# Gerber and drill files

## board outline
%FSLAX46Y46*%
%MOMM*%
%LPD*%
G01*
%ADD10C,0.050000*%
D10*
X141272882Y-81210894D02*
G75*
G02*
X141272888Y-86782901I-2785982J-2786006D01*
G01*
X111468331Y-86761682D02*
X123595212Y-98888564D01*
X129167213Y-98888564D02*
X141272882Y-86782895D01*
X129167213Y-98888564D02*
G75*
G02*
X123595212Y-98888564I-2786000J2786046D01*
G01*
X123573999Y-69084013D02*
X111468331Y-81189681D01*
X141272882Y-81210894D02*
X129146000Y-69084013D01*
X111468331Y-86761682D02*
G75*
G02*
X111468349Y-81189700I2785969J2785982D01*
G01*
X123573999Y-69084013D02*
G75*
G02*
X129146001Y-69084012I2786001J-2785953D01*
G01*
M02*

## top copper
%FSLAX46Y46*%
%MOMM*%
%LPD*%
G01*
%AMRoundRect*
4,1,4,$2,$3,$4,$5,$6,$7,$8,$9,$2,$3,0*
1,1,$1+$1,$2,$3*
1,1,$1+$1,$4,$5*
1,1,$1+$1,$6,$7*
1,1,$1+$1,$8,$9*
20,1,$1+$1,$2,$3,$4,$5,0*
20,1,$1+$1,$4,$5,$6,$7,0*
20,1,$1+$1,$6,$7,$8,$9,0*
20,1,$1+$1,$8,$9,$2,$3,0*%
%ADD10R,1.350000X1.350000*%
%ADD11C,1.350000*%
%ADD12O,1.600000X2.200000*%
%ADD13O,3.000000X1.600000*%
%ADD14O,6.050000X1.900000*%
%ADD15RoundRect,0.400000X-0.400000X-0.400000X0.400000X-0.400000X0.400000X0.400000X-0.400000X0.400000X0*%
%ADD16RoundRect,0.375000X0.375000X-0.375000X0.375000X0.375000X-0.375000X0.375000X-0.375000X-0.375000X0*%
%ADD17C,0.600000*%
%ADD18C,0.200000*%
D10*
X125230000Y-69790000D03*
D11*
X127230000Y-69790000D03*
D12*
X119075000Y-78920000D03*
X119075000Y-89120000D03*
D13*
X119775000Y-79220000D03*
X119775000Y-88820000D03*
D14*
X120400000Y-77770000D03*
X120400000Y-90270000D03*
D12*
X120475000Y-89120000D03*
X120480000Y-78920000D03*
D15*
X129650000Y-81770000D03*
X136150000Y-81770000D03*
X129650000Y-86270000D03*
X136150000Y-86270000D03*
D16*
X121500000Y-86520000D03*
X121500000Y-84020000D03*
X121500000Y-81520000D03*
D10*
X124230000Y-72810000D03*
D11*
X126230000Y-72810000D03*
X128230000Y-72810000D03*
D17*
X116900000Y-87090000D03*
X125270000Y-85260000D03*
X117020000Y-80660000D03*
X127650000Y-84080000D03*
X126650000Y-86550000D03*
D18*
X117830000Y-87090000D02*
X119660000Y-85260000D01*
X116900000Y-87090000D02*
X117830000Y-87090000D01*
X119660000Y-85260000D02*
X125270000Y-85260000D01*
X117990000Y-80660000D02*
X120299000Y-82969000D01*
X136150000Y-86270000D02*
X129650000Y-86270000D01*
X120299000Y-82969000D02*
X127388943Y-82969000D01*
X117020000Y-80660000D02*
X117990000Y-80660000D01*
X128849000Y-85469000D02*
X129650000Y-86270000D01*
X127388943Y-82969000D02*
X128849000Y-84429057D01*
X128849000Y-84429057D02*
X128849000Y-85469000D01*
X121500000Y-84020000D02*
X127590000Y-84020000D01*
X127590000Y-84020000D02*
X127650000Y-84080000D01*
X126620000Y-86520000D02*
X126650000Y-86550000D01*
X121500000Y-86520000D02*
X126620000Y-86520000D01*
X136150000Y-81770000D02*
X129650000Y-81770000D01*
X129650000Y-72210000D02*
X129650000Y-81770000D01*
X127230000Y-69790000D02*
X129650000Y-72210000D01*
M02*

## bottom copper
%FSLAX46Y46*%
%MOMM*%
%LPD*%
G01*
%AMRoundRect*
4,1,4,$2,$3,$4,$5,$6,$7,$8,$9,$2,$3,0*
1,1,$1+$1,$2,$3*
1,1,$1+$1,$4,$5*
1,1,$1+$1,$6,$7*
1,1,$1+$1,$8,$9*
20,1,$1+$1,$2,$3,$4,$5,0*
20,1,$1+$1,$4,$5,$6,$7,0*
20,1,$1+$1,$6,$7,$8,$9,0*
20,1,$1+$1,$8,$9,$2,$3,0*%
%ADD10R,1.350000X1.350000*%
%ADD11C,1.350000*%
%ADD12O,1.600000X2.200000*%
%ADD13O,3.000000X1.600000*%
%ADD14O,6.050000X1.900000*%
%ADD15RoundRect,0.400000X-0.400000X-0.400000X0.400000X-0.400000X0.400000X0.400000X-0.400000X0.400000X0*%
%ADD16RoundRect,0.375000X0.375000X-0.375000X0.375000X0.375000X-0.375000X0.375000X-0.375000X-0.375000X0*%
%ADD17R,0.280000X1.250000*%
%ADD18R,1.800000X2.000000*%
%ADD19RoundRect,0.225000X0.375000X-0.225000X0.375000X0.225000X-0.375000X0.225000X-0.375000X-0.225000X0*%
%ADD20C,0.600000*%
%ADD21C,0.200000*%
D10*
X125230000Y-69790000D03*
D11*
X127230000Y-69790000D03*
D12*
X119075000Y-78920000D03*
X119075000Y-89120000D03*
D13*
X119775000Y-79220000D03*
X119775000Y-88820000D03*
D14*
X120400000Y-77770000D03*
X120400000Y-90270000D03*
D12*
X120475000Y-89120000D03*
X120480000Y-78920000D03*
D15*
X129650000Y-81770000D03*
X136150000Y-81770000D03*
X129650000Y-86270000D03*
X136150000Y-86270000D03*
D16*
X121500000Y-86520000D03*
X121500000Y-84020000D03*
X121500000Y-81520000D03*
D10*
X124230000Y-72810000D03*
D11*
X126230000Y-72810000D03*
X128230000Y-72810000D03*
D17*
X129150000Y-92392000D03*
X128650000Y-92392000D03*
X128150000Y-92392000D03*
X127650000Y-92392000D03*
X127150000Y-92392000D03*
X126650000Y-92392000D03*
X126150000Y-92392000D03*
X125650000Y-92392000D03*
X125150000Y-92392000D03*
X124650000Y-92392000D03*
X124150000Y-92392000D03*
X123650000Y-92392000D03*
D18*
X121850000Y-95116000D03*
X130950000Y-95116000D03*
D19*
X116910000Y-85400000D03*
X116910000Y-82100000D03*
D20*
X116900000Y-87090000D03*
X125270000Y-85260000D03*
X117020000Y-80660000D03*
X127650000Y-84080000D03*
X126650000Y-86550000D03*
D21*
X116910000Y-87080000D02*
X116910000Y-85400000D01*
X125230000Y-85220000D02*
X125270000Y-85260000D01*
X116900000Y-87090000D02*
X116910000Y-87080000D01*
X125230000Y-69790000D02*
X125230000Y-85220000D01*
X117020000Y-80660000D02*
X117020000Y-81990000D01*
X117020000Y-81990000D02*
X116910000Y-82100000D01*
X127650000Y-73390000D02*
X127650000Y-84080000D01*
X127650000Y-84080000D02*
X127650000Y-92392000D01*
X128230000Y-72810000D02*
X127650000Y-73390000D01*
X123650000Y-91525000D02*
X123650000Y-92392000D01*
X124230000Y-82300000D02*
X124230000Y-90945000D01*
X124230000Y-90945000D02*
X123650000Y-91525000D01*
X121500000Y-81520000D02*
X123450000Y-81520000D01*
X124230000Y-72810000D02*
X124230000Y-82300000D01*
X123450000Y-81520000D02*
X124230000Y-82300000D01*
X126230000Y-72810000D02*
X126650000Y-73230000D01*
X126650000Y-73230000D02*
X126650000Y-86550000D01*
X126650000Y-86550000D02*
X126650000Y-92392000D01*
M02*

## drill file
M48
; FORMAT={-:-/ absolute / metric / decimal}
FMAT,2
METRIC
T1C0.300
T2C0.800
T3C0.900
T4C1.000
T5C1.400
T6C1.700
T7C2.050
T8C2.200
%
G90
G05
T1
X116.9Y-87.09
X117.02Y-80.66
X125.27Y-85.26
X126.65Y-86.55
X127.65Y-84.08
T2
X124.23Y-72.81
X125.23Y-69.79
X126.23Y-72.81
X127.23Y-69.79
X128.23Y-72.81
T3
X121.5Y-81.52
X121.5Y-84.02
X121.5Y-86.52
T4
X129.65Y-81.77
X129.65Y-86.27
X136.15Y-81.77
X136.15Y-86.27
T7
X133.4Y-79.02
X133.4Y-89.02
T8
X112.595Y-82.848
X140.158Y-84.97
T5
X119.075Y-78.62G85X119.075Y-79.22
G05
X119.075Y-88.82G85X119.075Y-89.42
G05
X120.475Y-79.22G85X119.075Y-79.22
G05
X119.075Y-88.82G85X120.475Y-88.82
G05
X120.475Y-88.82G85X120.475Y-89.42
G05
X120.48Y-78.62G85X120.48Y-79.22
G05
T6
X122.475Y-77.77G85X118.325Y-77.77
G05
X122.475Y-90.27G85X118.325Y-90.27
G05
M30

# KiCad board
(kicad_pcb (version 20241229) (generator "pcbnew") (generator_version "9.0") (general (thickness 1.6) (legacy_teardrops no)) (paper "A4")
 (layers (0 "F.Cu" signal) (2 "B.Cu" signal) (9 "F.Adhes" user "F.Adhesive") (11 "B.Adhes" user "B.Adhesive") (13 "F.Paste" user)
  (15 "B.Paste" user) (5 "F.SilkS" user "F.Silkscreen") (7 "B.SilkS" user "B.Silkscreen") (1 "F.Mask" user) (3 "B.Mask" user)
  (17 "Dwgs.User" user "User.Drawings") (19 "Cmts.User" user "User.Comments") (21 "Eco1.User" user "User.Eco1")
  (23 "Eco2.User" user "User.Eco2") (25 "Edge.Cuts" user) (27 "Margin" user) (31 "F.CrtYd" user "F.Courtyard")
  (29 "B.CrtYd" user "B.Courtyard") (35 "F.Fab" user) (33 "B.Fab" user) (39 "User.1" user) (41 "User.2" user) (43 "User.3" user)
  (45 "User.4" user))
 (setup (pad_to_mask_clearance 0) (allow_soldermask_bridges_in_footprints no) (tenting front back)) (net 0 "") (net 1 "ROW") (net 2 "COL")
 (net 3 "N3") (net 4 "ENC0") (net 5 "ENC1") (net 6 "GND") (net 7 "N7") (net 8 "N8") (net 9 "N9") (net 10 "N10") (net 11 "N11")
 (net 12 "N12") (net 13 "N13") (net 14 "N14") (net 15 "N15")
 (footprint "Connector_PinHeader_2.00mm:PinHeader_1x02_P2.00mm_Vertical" (layer "F.Cu") (at 125.23 69.79 90)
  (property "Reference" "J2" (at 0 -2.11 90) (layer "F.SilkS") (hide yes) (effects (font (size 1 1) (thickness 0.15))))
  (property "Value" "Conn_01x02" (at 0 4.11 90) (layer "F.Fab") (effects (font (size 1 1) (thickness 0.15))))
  (pad "1" thru_hole rect (at 0 0 90) (size 1.35 1.35) (drill 0.8) (layers "*.Cu" "*.Mask") (remove_unused_layers no) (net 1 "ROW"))
  (pad "2" thru_hole circle (at 0 2 90) (size 1.35 1.35) (drill 0.8) (layers "*.Cu" "*.Mask") (remove_unused_layers no) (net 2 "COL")))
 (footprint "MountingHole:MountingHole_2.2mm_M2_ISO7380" (layer "F.Cu") (at 112.595129 82.848498 45)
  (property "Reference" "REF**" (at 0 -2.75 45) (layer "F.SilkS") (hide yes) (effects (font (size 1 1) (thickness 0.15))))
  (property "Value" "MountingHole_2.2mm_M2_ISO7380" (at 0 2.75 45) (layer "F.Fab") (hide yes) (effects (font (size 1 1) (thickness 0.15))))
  (pad "" np_thru_hole circle (at 0 0 45) (size 2.2 2.2) (drill 2.2) (layers "*.Cu" "*.Mask")))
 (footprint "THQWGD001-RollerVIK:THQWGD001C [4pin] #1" (layer "F.Cu") (at 126.4 84.02)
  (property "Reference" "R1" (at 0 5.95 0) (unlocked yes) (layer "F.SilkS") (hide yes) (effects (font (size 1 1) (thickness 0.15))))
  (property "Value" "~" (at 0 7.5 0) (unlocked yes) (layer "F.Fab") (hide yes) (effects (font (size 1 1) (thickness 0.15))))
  (pad "" thru_hole oval (at -7.325 -5.1 270) (size 2.2 1.6) (drill oval 2 1.4) (layers "*.Cu" "*.Mask") (remove_unused_layers no))
  (pad "" thru_hole oval (at -7.325 5.1 270) (size 2.2 1.6) (drill oval 2 1.4) (layers "*.Cu" "*.Mask") (remove_unused_layers no))
  (pad "" thru_hole oval (at -6.625 -4.8 180) (size 3 1.6) (drill oval 2.8 1.4) (layers "*.Cu" "*.Mask") (remove_unused_layers no))
  (pad "" thru_hole oval (at -6.625 4.8) (size 3 1.6) (drill oval 2.8 1.4) (layers "*.Cu" "*.Mask") (remove_unused_layers no))
  (pad "" thru_hole oval (at -6 -6.25 270) (size 1.9 6.05) (drill oval 1.7 5.85) (layers "*.Cu" "*.Mask") (remove_unused_layers no))
  (pad "" thru_hole oval (at -6 6.25 270) (size 1.9 6.05) (drill oval 1.7 5.85) (layers "*.Cu" "*.Mask") (remove_unused_layers no))
  (pad "" thru_hole oval (at -5.925 5.1 270) (size 2.2 1.6) (drill oval 2 1.4) (layers "*.Cu" "*.Mask") (remove_unused_layers no))
  (pad "" thru_hole oval (at -5.92 -5.1 270) (size 2.2 1.6) (drill oval 2 1.4) (layers "*.Cu" "*.Mask") (remove_unused_layers no))
  (pad "" np_thru_hole circle (at 7 -5) (size 2.05 2.05) (drill 2.05) (layers "*.Cu" "*.Mask"))
  (pad "" np_thru_hole circle (at 7 5) (size 2.05 2.05) (drill 2.05) (layers "*.Cu" "*.Mask"))
  (pad "1" thru_hole roundrect (at 3.25 -2.25) (size 1.6 1.6) (drill 1) (layers "*.Cu" "B.Mask") (remove_unused_layers no)
   (roundrect_rratio 0.25) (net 2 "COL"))
  (pad "1" thru_hole roundrect (at 9.75 -2.25) (size 1.6 1.6) (drill 1) (layers "*.Cu" "B.Mask") (remove_unused_layers no)
   (roundrect_rratio 0.25) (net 2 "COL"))
  (pad "2" thru_hole roundrect (at 3.25 2.25) (size 1.6 1.6) (drill 1) (layers "*.Cu" "B.Mask") (remove_unused_layers no)
   (roundrect_rratio 0.25) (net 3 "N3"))
  (pad "2" thru_hole roundrect (at 9.75 2.25) (size 1.6 1.6) (drill 1) (layers "*.Cu" "B.Mask") (remove_unused_layers no)
   (roundrect_rratio 0.25) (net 3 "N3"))
  (pad "A" thru_hole roundrect (at -4.9 2.5 90) (size 1.5 1.5) (drill 0.9) (layers "*.Cu" "B.Mask") (remove_unused_layers no)
   (roundrect_rratio 0.25) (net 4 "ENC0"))
  (pad "B" thru_hole roundrect (at -4.9 0 90) (size 1.5 1.5) (drill 0.9) (layers "*.Cu" "B.Mask") (remove_unused_layers no)
   (roundrect_rratio 0.25) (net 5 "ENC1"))
  (pad "C" thru_hole roundrect (at -4.9 -2.5 90) (size 1.5 1.5) (drill 0.9) (layers "*.Cu" "B.Mask") (remove_unused_layers no)
   (roundrect_rratio 0.25) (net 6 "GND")))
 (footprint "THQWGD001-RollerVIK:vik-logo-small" (layer "F.Cu") (at 126.46 85.39)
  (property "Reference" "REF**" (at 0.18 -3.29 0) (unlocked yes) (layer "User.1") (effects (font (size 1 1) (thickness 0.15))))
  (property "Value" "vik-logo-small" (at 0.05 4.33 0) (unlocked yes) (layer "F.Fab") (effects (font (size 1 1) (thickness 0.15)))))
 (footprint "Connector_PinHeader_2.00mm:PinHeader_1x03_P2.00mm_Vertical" (layer "F.Cu") (at 124.23 72.81 90)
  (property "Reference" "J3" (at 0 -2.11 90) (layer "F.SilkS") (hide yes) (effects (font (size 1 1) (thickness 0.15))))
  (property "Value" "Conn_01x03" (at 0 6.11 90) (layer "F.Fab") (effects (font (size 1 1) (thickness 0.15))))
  (pad "1" thru_hole rect (at 0 0 90) (size 1.35 1.35) (drill 0.8) (layers "*.Cu" "*.Mask") (remove_unused_layers no) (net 6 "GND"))
  (pad "2" thru_hole circle (at 0 2 90) (size 1.35 1.35) (drill 0.8) (layers "*.Cu" "*.Mask") (remove_unused_layers no) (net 4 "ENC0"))
  (pad "3" thru_hole circle (at 0 4 90) (size 1.35 1.35) (drill 0.8) (layers "*.Cu" "*.Mask") (remove_unused_layers no) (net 5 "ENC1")))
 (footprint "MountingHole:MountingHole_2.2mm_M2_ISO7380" (layer "F.Cu") (at 140.158152 84.969818 135)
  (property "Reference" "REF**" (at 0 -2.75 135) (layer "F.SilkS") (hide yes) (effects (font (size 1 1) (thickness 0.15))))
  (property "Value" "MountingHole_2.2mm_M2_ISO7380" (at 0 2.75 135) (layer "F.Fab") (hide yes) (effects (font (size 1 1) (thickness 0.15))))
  (pad "" np_thru_hole circle (at 0 0 135) (size 2.2 2.2) (drill 2.2) (layers "*.Cu" "*.Mask")))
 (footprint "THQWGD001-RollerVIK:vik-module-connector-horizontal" (layer "B.Cu") (at 126.4 94.43 180)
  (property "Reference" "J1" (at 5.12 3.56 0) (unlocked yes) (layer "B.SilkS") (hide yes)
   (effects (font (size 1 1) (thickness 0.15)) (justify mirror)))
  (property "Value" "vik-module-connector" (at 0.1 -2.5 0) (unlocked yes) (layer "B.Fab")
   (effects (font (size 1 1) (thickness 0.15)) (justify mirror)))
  (pad "1" smd rect (at -2.75 2.038 180) (size 0.28 1.25) (layers "B.Cu" "B.Mask" "B.Paste") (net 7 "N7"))
  (pad "2" smd rect (at -2.25 2.038 180) (size 0.28 1.25) (layers "B.Cu" "B.Mask" "B.Paste") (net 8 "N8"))
  (pad "3" smd rect (at -1.75 2.038 180) (size 0.28 1.25) (layers "B.Cu" "B.Mask" "B.Paste") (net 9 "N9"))
  (pad "4" smd rect (at -1.25 2.038 180) (size 0.28 1.25) (layers "B.Cu" "B.Mask" "B.Paste") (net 5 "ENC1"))
  (pad "5" smd rect (at -0.75 2.038 180) (size 0.28 1.25) (layers "B.Cu" "B.Mask" "B.Paste") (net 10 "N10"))
  (pad "6" smd rect (at -0.25 2.038 180) (size 0.28 1.25) (layers "B.Cu" "B.Mask" "B.Paste") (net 4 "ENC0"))
  (pad "7" smd rect (at 0.25 2.038 180) (size 0.28 1.25) (layers "B.Cu" "B.Mask" "B.Paste") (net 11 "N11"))
  (pad "8" smd rect (at 0.75 2.038 180) (size 0.28 1.25) (layers "B.Cu" "B.Mask" "B.Paste") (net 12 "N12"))
  (pad "9" smd rect (at 1.25 2.038 180) (size 0.28 1.25) (layers "B.Cu" "B.Mask" "B.Paste") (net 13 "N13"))
  (pad "10" smd rect (at 1.75 2.038 180) (size 0.28 1.25) (layers "B.Cu" "B.Mask" "B.Paste") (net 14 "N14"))
  (pad "11" smd rect (at 2.25 2.038 180) (size 0.28 1.25) (layers "B.Cu" "B.Mask" "B.Paste") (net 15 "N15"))
  (pad "12" smd rect (at 2.75 2.038 180) (size 0.28 1.25) (layers "B.Cu" "B.Mask" "B.Paste") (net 6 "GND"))
  (pad "13" smd rect (at 4.55 -0.686 180) (size 1.8 2) (layers "B.Cu" "B.Mask" "B.Paste"))
  (pad "14" smd rect (at -4.55 -0.686 180) (size 1.8 2) (layers "B.Cu" "B.Mask" "B.Paste")))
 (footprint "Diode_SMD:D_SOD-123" (layer "B.Cu") (at 116.91 83.75 90)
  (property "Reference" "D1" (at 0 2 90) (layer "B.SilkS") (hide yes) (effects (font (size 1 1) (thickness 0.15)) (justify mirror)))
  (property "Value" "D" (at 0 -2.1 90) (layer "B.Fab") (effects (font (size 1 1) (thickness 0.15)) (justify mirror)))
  (pad "1" smd roundrect (at -1.65 0 90) (size 0.9 1.2) (layers "B.Cu" "B.Mask" "B.Paste") (roundrect_rratio 0.25) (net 1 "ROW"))
  (pad "2" smd roundrect (at 1.65 0 90) (size 0.9 1.2) (layers "B.Cu" "B.Mask" "B.Paste") (roundrect_rratio 0.25) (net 3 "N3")))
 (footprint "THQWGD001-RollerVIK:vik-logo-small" (layer "B.Cu") (at 126.46 85.39 180)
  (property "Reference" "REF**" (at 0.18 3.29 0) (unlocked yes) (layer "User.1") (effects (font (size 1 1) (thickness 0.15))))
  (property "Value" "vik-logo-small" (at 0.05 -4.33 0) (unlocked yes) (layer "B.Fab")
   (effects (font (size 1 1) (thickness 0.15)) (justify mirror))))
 (gr_arc (start 141.272882 81.210894) (mid 142.4269 83.996895) (end 141.272882 86.782895) (stroke (width 0.05) (type solid))
  (layer "Edge.Cuts"))
 (gr_line (start 111.468331 86.761682) (end 123.595212 98.888564) (stroke (width 0.05) (type solid)) (layer "Edge.Cuts"))
 (gr_line (start 129.167213 98.888564) (end 141.272882 86.782895) (stroke (width 0.05) (type solid)) (layer "Edge.Cuts"))
 (gr_arc (start 129.167213 98.888564) (mid 126.381213 100.04255) (end 123.595212 98.888564) (stroke (width 0.05) (type solid))
  (layer "Edge.Cuts"))
 (gr_line (start 123.573999 69.084013) (end 111.468331 81.189681) (stroke (width 0.05) (type solid)) (layer "Edge.Cuts"))
 (gr_line (start 141.272882 81.210894) (end 129.146 69.084013) (stroke (width 0.05) (type solid)) (layer "Edge.Cuts"))
 (gr_arc (start 111.468331 86.761682) (mid 110.314332 83.975682) (end 111.468331 81.189681) (stroke (width 0.05) (type solid))
  (layer "Edge.Cuts"))
 (gr_arc (start 123.573999 69.084013) (mid 126.36 67.93) (end 129.146 69.084013) (stroke (width 0.05) (type solid)) (layer "Edge.Cuts"))
 (segment (start 117.83 87.09) (end 119.66 85.26) (width 0.2) (layer "F.Cu") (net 1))
 (segment (start 116.9 87.09) (end 117.83 87.09) (width 0.2) (layer "F.Cu") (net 1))
 (segment (start 119.66 85.26) (end 125.27 85.26) (width 0.2) (layer "F.Cu") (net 1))
 (via (at 116.9 87.09) (size 0.6) (drill 0.3) (layers "F.Cu" "B.Cu") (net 1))
 (via (at 125.27 85.26) (size 0.6) (drill 0.3) (layers "F.Cu" "B.Cu") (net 1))
 (segment (start 116.91 87.08) (end 116.91 85.4) (width 0.2) (layer "B.Cu") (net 1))
 (segment (start 125.23 85.22) (end 125.27 85.26) (width 0.2) (layer "B.Cu") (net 1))
 (segment (start 116.9 87.09) (end 116.91 87.08) (width 0.2) (layer "B.Cu") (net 1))
 (segment (start 125.23 69.79) (end 125.23 85.22) (width 0.2) (layer "B.Cu") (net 1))
 (segment (start 117.99 80.66) (end 120.299 82.969) (width 0.2) (layer "F.Cu") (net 3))
 (segment (start 136.15 86.27) (end 129.65 86.27) (width 0.2) (layer "F.Cu") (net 3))
 (segment (start 120.299 82.969) (end 127.388943 82.969) (width 0.2) (layer "F.Cu") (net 3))
 (segment (start 117.02 80.66) (end 117.99 80.66) (width 0.2) (layer "F.Cu") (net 3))
 (segment (start 128.849 85.469) (end 129.65 86.27) (width 0.2) (layer "F.Cu") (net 3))
 (segment (start 127.388943 82.969) (end 128.849 84.429057) (width 0.2) (layer "F.Cu") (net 3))
 (segment (start 128.849 84.429057) (end 128.849 85.469) (width 0.2) (layer "F.Cu") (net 3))
 (via (at 117.02 80.66) (size 0.6) (drill 0.3) (layers "F.Cu" "B.Cu") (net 3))
 (segment (start 117.02 80.66) (end 117.02 81.99) (width 0.2) (layer "B.Cu") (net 3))
 (segment (start 117.02 81.99) (end 116.91 82.1) (width 0.2) (layer "B.Cu") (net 3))
 (segment (start 121.5 84.02) (end 127.59 84.02) (width 0.2) (layer "F.Cu") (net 5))
 (segment (start 127.59 84.02) (end 127.65 84.08) (width 0.2) (layer "F.Cu") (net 5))
 (via (at 127.65 84.08) (size 0.6) (drill 0.3) (layers "F.Cu" "B.Cu") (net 5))
 (segment (start 127.65 73.39) (end 127.65 84.08) (width 0.2) (layer "B.Cu") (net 5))
 (segment (start 127.65 84.08) (end 127.65 92.392) (width 0.2) (layer "B.Cu") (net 5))
 (segment (start 128.23 72.81) (end 127.65 73.39) (width 0.2) (layer "B.Cu") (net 5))
 (segment (start 123.65 91.525) (end 123.65 92.392) (width 0.2) (layer "B.Cu") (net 6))
 (segment (start 124.23 82.3) (end 124.23 90.945) (width 0.2) (layer "B.Cu") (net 6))
 (segment (start 124.23 90.945) (end 123.65 91.525) (width 0.2) (layer "B.Cu") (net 6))
 (segment (start 121.5 81.52) (end 123.45 81.52) (width 0.2) (layer "B.Cu") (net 6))
 (segment (start 124.23 72.81) (end 124.23 82.3) (width 0.2) (layer "B.Cu") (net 6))
 (segment (start 123.45 81.52) (end 124.23 82.3) (width 0.2) (layer "B.Cu") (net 6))
 (segment (start 126.62 86.52) (end 126.65 86.55) (width 0.2) (layer "F.Cu") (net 4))
 (segment (start 121.5 86.52) (end 126.62 86.52) (width 0.2) (layer "F.Cu") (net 4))
 (via (at 126.65 86.55) (size 0.6) (drill 0.3) (layers "F.Cu" "B.Cu") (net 4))
 (segment (start 126.23 72.81) (end 126.65 73.23) (width 0.2) (layer "B.Cu") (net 4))
 (segment (start 126.65 73.23) (end 126.65 86.55) (width 0.2) (layer "B.Cu") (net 4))
 (segment (start 126.65 86.55) (end 126.65 92.392) (width 0.2) (layer "B.Cu") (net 4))
 (segment (start 136.15 81.77) (end 129.65 81.77) (width 0.2) (layer "F.Cu") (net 2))
 (segment (start 129.65 72.21) (end 129.65 81.77) (width 0.2) (layer "F.Cu") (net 2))
 (segment (start 127.23 69.79) (end 129.65 72.21) (width 0.2) (layer "F.Cu") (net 2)))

